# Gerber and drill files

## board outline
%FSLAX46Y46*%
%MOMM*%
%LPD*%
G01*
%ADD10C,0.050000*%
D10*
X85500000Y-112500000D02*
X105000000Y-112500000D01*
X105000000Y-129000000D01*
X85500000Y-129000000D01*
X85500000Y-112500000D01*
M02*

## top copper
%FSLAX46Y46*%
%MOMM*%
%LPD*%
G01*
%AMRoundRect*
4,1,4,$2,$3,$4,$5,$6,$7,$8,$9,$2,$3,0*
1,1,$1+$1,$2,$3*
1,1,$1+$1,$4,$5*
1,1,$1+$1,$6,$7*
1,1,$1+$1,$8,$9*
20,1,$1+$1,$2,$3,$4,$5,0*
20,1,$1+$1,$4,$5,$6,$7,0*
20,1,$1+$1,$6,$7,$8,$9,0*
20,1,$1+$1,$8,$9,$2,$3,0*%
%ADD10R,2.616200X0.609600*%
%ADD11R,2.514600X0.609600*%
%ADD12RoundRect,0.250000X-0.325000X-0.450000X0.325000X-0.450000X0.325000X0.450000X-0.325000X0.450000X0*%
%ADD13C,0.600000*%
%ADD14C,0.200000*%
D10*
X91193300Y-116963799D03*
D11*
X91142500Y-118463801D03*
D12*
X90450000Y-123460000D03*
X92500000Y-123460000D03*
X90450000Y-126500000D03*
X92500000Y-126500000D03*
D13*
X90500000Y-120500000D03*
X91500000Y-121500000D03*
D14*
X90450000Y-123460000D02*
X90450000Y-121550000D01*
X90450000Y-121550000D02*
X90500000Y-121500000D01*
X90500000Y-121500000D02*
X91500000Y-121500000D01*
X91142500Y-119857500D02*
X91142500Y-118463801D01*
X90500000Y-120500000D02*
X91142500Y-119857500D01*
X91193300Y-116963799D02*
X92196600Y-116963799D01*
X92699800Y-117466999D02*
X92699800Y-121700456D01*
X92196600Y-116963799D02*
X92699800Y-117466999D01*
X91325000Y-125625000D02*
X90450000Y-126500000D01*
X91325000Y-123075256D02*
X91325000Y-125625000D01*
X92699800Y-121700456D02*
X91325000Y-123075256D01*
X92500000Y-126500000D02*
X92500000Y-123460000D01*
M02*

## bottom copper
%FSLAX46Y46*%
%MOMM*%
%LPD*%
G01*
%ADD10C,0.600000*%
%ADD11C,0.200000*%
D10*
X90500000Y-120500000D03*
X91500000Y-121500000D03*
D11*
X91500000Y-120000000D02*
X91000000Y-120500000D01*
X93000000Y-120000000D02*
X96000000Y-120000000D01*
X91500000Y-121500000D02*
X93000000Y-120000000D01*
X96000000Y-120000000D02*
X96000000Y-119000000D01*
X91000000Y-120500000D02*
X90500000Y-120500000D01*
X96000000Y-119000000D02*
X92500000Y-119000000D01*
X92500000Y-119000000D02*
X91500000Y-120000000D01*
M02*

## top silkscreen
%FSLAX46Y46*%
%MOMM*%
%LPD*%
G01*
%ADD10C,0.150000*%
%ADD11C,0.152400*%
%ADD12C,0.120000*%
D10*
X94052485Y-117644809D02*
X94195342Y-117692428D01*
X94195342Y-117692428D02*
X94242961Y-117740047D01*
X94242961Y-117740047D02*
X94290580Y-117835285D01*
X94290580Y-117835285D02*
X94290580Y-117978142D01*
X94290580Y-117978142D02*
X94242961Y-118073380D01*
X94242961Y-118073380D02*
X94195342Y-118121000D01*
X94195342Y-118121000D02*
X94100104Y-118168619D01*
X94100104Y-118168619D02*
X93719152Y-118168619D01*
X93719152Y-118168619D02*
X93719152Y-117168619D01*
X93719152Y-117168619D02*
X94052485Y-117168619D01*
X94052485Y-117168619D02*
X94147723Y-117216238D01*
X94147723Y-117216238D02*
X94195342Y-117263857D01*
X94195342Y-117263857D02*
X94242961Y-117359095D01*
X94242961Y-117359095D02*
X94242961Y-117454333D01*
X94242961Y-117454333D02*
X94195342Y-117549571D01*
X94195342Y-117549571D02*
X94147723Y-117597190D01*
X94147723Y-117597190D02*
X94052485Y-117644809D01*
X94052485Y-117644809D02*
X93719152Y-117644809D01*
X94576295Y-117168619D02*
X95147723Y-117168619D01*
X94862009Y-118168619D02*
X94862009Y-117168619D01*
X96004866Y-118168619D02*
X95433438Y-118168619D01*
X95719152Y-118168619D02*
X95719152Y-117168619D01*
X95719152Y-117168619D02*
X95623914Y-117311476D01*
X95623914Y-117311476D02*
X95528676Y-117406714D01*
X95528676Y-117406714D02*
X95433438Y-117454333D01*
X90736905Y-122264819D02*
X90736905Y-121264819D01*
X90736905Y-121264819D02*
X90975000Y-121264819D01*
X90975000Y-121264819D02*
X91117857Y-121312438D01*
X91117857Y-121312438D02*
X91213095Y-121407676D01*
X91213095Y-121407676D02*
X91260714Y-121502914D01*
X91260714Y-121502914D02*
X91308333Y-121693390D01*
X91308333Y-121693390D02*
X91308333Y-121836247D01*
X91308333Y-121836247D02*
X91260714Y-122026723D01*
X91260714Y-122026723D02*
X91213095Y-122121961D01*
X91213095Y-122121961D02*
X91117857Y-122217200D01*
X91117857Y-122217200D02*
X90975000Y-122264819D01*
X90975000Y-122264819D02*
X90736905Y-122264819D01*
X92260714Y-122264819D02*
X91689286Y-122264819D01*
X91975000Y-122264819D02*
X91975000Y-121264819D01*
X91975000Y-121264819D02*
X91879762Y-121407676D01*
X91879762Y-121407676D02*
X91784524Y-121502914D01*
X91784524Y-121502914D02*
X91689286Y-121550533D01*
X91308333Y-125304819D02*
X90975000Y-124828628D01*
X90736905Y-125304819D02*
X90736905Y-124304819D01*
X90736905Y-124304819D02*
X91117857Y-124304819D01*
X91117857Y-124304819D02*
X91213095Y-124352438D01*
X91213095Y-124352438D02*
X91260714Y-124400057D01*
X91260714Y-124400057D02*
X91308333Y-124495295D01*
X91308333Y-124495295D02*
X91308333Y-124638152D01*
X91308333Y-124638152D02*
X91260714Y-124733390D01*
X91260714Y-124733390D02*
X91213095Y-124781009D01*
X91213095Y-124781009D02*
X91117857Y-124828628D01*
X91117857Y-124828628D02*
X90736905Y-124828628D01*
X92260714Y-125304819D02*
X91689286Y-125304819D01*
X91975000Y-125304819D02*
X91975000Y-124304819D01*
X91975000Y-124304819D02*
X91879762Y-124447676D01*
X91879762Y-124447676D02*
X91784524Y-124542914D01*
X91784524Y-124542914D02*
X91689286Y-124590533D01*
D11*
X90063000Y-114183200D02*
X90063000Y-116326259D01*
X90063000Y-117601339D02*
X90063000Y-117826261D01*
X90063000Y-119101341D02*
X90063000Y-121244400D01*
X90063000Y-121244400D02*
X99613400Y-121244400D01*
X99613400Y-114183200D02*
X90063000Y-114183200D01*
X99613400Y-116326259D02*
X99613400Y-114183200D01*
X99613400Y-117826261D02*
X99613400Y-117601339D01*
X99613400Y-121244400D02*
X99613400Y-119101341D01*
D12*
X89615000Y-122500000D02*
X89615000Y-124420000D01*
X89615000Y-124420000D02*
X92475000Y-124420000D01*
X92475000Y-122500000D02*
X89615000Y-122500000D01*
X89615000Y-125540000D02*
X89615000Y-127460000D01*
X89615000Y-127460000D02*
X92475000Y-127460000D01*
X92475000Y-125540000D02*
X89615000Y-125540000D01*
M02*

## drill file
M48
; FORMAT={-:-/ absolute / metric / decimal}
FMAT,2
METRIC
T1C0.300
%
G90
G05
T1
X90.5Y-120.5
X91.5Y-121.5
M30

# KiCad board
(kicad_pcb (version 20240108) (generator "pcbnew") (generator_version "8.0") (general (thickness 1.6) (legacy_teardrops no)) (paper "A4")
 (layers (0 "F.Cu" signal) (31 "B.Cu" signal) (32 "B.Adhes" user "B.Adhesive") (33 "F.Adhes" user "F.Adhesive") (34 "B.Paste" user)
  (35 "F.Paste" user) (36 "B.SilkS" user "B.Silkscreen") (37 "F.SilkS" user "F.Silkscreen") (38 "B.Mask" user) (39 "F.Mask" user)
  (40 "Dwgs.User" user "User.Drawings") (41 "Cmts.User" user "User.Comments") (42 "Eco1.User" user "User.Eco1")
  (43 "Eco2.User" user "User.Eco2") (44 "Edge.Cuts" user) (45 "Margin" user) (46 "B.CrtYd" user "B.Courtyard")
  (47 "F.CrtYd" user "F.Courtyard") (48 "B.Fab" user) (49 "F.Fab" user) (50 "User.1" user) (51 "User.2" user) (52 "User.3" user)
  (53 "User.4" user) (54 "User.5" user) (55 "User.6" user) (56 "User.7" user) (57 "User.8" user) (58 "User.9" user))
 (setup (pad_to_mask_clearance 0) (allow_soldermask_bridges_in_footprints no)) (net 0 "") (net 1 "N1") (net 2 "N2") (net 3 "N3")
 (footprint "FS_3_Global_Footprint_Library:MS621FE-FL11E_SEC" (layer "F.Cu") (at 94.8382 117.7138)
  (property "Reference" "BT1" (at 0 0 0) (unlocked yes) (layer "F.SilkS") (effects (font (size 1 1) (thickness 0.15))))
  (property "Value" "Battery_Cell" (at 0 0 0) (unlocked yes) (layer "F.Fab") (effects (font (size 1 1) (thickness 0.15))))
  (fp_line (start -4.7752 -3.5306) (end -4.7752 -1.387541) (stroke (width 0.1524) (type solid)) (layer "F.SilkS"))
  (fp_line (start -4.7752 -0.112461) (end -4.7752 0.112461) (stroke (width 0.1524) (type solid)) (layer "F.SilkS"))
  (fp_line (start -4.7752 1.387541) (end -4.7752 3.5306) (stroke (width 0.1524) (type solid)) (layer "F.SilkS"))
  (fp_line (start -4.7752 3.5306) (end 4.7752 3.5306) (stroke (width 0.1524) (type solid)) (layer "F.SilkS"))
  (fp_line (start 4.7752 -3.5306) (end -4.7752 -3.5306) (stroke (width 0.1524) (type solid)) (layer "F.SilkS"))
  (fp_line (start 4.7752 -1.387541) (end 4.7752 -3.5306) (stroke (width 0.1524) (type solid)) (layer "F.SilkS"))
  (fp_line (start 4.7752 0.112461) (end 4.7752 -0.112461) (stroke (width 0.1524) (type solid)) (layer "F.SilkS"))
  (fp_line (start 4.7752 3.5306) (end 4.7752 1.387541) (stroke (width 0.1524) (type solid)) (layer "F.SilkS"))
  (pad "1" smd rect (at -3.6449 -0.750001) (size 2.6162 0.6096) (layers "F.Cu" "F.Paste" "F.Mask") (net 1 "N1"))
  (pad "2" smd rect (at -3.6957 0.750001) (size 2.5146 0.6096) (layers "F.Cu" "F.Paste" "F.Mask") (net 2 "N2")))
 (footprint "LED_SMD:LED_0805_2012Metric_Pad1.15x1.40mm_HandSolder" (layer "F.Cu") (at 91.475 123.46)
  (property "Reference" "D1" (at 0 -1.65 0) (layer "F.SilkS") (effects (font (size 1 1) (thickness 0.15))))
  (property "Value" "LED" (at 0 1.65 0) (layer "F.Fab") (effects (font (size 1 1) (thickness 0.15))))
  (fp_line (start -1.86 -0.96) (end -1.86 0.96) (stroke (width 0.12) (type solid)) (layer "F.SilkS"))
  (fp_line (start -1.86 0.96) (end 1 0.96) (stroke (width 0.12) (type solid)) (layer "F.SilkS"))
  (fp_line (start 1 -0.96) (end -1.86 -0.96) (stroke (width 0.12) (type solid)) (layer "F.SilkS"))
  (pad "1" smd roundrect (at -1.025 0) (size 1.15 1.4) (layers "F.Cu" "F.Paste" "F.Mask") (roundrect_rratio 0.217391) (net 2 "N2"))
  (pad "2" smd roundrect (at 1.025 0) (size 1.15 1.4) (layers "F.Cu" "F.Paste" "F.Mask") (roundrect_rratio 0.217391) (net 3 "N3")))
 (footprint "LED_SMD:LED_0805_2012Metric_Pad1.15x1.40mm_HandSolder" (layer "F.Cu") (at 91.475 126.5)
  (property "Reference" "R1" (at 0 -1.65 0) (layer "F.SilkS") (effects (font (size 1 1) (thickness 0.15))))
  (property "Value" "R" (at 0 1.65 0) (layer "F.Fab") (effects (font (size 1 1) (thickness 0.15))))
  (fp_line (start -1.86 -0.96) (end -1.86 0.96) (stroke (width 0.12) (type solid)) (layer "F.SilkS"))
  (fp_line (start -1.86 0.96) (end 1 0.96) (stroke (width 0.12) (type solid)) (layer "F.SilkS"))
  (fp_line (start 1 -0.96) (end -1.86 -0.96) (stroke (width 0.12) (type solid)) (layer "F.SilkS"))
  (pad "1" smd roundrect (at -1.025 0) (size 1.15 1.4) (layers "F.Cu" "F.Paste" "F.Mask") (roundrect_rratio 0.217391) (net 1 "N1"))
  (pad "2" smd roundrect (at 1.025 0) (size 1.15 1.4) (layers "F.Cu" "F.Paste" "F.Mask") (roundrect_rratio 0.217391) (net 3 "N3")))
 (gr_rect (start 85.5 112.5) (end 105 129) (stroke (width 0.05) (type default)) (fill none) (layer "Edge.Cuts"))
 (segment (start 90.45 123.46) (end 90.45 121.55) (width 0.2) (layer "F.Cu") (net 2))
 (segment (start 90.45 121.55) (end 90.5 121.5) (width 0.2) (layer "F.Cu") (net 2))
 (segment (start 90.5 121.5) (end 91.5 121.5) (width 0.2) (layer "F.Cu") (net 2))
 (segment (start 91.1425 119.8575) (end 91.1425 118.463801) (width 0.2) (layer "F.Cu") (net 2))
 (segment (start 90.5 120.5) (end 91.1425 119.8575) (width 0.2) (layer "F.Cu") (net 2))
 (via (at 90.5 120.5) (size 0.6) (drill 0.3) (layers "F.Cu" "B.Cu") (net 2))
 (via (at 91.5 121.5) (size 0.6) (drill 0.3) (layers "F.Cu" "B.Cu") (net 2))
 (segment (start 91.5 120) (end 91 120.5) (width 0.2) (layer "B.Cu") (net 2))
 (segment (start 93 120) (end 96 120) (width 0.2) (layer "B.Cu") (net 2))
 (segment (start 91.5 121.5) (end 93 120) (width 0.2) (layer "B.Cu") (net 2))
 (segment (start 96 120) (end 96 119) (width 0.2) (layer "B.Cu") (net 2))
 (segment (start 91 120.5) (end 90.5 120.5) (width 0.2) (layer "B.Cu") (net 2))
 (segment (start 96 119) (end 92.5 119) (width 0.2) (layer "B.Cu") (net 2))
 (segment (start 92.5 119) (end 91.5 120) (width 0.2) (layer "B.Cu") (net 2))
 (segment (start 91.1933 116.963799) (end 92.1966 116.963799) (width 0.2) (layer "F.Cu") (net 1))
 (segment (start 92.6998 117.466999) (end 92.6998 121.700456) (width 0.2) (layer "F.Cu") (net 1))
 (segment (start 92.1966 116.963799) (end 92.6998 117.466999) (width 0.2) (layer "F.Cu") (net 1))
 (segment (start 91.325 125.625) (end 90.45 126.5) (width 0.2) (layer "F.Cu") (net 1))
 (segment (start 91.325 123.075256) (end 91.325 125.625) (width 0.2) (layer "F.Cu") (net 1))
 (segment (start 92.6998 121.700456) (end 91.325 123.075256) (width 0.2) (layer "F.Cu") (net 1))
 (segment (start 92.5 126.5) (end 92.5 123.46) (width 0.2) (layer "F.Cu") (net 3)))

